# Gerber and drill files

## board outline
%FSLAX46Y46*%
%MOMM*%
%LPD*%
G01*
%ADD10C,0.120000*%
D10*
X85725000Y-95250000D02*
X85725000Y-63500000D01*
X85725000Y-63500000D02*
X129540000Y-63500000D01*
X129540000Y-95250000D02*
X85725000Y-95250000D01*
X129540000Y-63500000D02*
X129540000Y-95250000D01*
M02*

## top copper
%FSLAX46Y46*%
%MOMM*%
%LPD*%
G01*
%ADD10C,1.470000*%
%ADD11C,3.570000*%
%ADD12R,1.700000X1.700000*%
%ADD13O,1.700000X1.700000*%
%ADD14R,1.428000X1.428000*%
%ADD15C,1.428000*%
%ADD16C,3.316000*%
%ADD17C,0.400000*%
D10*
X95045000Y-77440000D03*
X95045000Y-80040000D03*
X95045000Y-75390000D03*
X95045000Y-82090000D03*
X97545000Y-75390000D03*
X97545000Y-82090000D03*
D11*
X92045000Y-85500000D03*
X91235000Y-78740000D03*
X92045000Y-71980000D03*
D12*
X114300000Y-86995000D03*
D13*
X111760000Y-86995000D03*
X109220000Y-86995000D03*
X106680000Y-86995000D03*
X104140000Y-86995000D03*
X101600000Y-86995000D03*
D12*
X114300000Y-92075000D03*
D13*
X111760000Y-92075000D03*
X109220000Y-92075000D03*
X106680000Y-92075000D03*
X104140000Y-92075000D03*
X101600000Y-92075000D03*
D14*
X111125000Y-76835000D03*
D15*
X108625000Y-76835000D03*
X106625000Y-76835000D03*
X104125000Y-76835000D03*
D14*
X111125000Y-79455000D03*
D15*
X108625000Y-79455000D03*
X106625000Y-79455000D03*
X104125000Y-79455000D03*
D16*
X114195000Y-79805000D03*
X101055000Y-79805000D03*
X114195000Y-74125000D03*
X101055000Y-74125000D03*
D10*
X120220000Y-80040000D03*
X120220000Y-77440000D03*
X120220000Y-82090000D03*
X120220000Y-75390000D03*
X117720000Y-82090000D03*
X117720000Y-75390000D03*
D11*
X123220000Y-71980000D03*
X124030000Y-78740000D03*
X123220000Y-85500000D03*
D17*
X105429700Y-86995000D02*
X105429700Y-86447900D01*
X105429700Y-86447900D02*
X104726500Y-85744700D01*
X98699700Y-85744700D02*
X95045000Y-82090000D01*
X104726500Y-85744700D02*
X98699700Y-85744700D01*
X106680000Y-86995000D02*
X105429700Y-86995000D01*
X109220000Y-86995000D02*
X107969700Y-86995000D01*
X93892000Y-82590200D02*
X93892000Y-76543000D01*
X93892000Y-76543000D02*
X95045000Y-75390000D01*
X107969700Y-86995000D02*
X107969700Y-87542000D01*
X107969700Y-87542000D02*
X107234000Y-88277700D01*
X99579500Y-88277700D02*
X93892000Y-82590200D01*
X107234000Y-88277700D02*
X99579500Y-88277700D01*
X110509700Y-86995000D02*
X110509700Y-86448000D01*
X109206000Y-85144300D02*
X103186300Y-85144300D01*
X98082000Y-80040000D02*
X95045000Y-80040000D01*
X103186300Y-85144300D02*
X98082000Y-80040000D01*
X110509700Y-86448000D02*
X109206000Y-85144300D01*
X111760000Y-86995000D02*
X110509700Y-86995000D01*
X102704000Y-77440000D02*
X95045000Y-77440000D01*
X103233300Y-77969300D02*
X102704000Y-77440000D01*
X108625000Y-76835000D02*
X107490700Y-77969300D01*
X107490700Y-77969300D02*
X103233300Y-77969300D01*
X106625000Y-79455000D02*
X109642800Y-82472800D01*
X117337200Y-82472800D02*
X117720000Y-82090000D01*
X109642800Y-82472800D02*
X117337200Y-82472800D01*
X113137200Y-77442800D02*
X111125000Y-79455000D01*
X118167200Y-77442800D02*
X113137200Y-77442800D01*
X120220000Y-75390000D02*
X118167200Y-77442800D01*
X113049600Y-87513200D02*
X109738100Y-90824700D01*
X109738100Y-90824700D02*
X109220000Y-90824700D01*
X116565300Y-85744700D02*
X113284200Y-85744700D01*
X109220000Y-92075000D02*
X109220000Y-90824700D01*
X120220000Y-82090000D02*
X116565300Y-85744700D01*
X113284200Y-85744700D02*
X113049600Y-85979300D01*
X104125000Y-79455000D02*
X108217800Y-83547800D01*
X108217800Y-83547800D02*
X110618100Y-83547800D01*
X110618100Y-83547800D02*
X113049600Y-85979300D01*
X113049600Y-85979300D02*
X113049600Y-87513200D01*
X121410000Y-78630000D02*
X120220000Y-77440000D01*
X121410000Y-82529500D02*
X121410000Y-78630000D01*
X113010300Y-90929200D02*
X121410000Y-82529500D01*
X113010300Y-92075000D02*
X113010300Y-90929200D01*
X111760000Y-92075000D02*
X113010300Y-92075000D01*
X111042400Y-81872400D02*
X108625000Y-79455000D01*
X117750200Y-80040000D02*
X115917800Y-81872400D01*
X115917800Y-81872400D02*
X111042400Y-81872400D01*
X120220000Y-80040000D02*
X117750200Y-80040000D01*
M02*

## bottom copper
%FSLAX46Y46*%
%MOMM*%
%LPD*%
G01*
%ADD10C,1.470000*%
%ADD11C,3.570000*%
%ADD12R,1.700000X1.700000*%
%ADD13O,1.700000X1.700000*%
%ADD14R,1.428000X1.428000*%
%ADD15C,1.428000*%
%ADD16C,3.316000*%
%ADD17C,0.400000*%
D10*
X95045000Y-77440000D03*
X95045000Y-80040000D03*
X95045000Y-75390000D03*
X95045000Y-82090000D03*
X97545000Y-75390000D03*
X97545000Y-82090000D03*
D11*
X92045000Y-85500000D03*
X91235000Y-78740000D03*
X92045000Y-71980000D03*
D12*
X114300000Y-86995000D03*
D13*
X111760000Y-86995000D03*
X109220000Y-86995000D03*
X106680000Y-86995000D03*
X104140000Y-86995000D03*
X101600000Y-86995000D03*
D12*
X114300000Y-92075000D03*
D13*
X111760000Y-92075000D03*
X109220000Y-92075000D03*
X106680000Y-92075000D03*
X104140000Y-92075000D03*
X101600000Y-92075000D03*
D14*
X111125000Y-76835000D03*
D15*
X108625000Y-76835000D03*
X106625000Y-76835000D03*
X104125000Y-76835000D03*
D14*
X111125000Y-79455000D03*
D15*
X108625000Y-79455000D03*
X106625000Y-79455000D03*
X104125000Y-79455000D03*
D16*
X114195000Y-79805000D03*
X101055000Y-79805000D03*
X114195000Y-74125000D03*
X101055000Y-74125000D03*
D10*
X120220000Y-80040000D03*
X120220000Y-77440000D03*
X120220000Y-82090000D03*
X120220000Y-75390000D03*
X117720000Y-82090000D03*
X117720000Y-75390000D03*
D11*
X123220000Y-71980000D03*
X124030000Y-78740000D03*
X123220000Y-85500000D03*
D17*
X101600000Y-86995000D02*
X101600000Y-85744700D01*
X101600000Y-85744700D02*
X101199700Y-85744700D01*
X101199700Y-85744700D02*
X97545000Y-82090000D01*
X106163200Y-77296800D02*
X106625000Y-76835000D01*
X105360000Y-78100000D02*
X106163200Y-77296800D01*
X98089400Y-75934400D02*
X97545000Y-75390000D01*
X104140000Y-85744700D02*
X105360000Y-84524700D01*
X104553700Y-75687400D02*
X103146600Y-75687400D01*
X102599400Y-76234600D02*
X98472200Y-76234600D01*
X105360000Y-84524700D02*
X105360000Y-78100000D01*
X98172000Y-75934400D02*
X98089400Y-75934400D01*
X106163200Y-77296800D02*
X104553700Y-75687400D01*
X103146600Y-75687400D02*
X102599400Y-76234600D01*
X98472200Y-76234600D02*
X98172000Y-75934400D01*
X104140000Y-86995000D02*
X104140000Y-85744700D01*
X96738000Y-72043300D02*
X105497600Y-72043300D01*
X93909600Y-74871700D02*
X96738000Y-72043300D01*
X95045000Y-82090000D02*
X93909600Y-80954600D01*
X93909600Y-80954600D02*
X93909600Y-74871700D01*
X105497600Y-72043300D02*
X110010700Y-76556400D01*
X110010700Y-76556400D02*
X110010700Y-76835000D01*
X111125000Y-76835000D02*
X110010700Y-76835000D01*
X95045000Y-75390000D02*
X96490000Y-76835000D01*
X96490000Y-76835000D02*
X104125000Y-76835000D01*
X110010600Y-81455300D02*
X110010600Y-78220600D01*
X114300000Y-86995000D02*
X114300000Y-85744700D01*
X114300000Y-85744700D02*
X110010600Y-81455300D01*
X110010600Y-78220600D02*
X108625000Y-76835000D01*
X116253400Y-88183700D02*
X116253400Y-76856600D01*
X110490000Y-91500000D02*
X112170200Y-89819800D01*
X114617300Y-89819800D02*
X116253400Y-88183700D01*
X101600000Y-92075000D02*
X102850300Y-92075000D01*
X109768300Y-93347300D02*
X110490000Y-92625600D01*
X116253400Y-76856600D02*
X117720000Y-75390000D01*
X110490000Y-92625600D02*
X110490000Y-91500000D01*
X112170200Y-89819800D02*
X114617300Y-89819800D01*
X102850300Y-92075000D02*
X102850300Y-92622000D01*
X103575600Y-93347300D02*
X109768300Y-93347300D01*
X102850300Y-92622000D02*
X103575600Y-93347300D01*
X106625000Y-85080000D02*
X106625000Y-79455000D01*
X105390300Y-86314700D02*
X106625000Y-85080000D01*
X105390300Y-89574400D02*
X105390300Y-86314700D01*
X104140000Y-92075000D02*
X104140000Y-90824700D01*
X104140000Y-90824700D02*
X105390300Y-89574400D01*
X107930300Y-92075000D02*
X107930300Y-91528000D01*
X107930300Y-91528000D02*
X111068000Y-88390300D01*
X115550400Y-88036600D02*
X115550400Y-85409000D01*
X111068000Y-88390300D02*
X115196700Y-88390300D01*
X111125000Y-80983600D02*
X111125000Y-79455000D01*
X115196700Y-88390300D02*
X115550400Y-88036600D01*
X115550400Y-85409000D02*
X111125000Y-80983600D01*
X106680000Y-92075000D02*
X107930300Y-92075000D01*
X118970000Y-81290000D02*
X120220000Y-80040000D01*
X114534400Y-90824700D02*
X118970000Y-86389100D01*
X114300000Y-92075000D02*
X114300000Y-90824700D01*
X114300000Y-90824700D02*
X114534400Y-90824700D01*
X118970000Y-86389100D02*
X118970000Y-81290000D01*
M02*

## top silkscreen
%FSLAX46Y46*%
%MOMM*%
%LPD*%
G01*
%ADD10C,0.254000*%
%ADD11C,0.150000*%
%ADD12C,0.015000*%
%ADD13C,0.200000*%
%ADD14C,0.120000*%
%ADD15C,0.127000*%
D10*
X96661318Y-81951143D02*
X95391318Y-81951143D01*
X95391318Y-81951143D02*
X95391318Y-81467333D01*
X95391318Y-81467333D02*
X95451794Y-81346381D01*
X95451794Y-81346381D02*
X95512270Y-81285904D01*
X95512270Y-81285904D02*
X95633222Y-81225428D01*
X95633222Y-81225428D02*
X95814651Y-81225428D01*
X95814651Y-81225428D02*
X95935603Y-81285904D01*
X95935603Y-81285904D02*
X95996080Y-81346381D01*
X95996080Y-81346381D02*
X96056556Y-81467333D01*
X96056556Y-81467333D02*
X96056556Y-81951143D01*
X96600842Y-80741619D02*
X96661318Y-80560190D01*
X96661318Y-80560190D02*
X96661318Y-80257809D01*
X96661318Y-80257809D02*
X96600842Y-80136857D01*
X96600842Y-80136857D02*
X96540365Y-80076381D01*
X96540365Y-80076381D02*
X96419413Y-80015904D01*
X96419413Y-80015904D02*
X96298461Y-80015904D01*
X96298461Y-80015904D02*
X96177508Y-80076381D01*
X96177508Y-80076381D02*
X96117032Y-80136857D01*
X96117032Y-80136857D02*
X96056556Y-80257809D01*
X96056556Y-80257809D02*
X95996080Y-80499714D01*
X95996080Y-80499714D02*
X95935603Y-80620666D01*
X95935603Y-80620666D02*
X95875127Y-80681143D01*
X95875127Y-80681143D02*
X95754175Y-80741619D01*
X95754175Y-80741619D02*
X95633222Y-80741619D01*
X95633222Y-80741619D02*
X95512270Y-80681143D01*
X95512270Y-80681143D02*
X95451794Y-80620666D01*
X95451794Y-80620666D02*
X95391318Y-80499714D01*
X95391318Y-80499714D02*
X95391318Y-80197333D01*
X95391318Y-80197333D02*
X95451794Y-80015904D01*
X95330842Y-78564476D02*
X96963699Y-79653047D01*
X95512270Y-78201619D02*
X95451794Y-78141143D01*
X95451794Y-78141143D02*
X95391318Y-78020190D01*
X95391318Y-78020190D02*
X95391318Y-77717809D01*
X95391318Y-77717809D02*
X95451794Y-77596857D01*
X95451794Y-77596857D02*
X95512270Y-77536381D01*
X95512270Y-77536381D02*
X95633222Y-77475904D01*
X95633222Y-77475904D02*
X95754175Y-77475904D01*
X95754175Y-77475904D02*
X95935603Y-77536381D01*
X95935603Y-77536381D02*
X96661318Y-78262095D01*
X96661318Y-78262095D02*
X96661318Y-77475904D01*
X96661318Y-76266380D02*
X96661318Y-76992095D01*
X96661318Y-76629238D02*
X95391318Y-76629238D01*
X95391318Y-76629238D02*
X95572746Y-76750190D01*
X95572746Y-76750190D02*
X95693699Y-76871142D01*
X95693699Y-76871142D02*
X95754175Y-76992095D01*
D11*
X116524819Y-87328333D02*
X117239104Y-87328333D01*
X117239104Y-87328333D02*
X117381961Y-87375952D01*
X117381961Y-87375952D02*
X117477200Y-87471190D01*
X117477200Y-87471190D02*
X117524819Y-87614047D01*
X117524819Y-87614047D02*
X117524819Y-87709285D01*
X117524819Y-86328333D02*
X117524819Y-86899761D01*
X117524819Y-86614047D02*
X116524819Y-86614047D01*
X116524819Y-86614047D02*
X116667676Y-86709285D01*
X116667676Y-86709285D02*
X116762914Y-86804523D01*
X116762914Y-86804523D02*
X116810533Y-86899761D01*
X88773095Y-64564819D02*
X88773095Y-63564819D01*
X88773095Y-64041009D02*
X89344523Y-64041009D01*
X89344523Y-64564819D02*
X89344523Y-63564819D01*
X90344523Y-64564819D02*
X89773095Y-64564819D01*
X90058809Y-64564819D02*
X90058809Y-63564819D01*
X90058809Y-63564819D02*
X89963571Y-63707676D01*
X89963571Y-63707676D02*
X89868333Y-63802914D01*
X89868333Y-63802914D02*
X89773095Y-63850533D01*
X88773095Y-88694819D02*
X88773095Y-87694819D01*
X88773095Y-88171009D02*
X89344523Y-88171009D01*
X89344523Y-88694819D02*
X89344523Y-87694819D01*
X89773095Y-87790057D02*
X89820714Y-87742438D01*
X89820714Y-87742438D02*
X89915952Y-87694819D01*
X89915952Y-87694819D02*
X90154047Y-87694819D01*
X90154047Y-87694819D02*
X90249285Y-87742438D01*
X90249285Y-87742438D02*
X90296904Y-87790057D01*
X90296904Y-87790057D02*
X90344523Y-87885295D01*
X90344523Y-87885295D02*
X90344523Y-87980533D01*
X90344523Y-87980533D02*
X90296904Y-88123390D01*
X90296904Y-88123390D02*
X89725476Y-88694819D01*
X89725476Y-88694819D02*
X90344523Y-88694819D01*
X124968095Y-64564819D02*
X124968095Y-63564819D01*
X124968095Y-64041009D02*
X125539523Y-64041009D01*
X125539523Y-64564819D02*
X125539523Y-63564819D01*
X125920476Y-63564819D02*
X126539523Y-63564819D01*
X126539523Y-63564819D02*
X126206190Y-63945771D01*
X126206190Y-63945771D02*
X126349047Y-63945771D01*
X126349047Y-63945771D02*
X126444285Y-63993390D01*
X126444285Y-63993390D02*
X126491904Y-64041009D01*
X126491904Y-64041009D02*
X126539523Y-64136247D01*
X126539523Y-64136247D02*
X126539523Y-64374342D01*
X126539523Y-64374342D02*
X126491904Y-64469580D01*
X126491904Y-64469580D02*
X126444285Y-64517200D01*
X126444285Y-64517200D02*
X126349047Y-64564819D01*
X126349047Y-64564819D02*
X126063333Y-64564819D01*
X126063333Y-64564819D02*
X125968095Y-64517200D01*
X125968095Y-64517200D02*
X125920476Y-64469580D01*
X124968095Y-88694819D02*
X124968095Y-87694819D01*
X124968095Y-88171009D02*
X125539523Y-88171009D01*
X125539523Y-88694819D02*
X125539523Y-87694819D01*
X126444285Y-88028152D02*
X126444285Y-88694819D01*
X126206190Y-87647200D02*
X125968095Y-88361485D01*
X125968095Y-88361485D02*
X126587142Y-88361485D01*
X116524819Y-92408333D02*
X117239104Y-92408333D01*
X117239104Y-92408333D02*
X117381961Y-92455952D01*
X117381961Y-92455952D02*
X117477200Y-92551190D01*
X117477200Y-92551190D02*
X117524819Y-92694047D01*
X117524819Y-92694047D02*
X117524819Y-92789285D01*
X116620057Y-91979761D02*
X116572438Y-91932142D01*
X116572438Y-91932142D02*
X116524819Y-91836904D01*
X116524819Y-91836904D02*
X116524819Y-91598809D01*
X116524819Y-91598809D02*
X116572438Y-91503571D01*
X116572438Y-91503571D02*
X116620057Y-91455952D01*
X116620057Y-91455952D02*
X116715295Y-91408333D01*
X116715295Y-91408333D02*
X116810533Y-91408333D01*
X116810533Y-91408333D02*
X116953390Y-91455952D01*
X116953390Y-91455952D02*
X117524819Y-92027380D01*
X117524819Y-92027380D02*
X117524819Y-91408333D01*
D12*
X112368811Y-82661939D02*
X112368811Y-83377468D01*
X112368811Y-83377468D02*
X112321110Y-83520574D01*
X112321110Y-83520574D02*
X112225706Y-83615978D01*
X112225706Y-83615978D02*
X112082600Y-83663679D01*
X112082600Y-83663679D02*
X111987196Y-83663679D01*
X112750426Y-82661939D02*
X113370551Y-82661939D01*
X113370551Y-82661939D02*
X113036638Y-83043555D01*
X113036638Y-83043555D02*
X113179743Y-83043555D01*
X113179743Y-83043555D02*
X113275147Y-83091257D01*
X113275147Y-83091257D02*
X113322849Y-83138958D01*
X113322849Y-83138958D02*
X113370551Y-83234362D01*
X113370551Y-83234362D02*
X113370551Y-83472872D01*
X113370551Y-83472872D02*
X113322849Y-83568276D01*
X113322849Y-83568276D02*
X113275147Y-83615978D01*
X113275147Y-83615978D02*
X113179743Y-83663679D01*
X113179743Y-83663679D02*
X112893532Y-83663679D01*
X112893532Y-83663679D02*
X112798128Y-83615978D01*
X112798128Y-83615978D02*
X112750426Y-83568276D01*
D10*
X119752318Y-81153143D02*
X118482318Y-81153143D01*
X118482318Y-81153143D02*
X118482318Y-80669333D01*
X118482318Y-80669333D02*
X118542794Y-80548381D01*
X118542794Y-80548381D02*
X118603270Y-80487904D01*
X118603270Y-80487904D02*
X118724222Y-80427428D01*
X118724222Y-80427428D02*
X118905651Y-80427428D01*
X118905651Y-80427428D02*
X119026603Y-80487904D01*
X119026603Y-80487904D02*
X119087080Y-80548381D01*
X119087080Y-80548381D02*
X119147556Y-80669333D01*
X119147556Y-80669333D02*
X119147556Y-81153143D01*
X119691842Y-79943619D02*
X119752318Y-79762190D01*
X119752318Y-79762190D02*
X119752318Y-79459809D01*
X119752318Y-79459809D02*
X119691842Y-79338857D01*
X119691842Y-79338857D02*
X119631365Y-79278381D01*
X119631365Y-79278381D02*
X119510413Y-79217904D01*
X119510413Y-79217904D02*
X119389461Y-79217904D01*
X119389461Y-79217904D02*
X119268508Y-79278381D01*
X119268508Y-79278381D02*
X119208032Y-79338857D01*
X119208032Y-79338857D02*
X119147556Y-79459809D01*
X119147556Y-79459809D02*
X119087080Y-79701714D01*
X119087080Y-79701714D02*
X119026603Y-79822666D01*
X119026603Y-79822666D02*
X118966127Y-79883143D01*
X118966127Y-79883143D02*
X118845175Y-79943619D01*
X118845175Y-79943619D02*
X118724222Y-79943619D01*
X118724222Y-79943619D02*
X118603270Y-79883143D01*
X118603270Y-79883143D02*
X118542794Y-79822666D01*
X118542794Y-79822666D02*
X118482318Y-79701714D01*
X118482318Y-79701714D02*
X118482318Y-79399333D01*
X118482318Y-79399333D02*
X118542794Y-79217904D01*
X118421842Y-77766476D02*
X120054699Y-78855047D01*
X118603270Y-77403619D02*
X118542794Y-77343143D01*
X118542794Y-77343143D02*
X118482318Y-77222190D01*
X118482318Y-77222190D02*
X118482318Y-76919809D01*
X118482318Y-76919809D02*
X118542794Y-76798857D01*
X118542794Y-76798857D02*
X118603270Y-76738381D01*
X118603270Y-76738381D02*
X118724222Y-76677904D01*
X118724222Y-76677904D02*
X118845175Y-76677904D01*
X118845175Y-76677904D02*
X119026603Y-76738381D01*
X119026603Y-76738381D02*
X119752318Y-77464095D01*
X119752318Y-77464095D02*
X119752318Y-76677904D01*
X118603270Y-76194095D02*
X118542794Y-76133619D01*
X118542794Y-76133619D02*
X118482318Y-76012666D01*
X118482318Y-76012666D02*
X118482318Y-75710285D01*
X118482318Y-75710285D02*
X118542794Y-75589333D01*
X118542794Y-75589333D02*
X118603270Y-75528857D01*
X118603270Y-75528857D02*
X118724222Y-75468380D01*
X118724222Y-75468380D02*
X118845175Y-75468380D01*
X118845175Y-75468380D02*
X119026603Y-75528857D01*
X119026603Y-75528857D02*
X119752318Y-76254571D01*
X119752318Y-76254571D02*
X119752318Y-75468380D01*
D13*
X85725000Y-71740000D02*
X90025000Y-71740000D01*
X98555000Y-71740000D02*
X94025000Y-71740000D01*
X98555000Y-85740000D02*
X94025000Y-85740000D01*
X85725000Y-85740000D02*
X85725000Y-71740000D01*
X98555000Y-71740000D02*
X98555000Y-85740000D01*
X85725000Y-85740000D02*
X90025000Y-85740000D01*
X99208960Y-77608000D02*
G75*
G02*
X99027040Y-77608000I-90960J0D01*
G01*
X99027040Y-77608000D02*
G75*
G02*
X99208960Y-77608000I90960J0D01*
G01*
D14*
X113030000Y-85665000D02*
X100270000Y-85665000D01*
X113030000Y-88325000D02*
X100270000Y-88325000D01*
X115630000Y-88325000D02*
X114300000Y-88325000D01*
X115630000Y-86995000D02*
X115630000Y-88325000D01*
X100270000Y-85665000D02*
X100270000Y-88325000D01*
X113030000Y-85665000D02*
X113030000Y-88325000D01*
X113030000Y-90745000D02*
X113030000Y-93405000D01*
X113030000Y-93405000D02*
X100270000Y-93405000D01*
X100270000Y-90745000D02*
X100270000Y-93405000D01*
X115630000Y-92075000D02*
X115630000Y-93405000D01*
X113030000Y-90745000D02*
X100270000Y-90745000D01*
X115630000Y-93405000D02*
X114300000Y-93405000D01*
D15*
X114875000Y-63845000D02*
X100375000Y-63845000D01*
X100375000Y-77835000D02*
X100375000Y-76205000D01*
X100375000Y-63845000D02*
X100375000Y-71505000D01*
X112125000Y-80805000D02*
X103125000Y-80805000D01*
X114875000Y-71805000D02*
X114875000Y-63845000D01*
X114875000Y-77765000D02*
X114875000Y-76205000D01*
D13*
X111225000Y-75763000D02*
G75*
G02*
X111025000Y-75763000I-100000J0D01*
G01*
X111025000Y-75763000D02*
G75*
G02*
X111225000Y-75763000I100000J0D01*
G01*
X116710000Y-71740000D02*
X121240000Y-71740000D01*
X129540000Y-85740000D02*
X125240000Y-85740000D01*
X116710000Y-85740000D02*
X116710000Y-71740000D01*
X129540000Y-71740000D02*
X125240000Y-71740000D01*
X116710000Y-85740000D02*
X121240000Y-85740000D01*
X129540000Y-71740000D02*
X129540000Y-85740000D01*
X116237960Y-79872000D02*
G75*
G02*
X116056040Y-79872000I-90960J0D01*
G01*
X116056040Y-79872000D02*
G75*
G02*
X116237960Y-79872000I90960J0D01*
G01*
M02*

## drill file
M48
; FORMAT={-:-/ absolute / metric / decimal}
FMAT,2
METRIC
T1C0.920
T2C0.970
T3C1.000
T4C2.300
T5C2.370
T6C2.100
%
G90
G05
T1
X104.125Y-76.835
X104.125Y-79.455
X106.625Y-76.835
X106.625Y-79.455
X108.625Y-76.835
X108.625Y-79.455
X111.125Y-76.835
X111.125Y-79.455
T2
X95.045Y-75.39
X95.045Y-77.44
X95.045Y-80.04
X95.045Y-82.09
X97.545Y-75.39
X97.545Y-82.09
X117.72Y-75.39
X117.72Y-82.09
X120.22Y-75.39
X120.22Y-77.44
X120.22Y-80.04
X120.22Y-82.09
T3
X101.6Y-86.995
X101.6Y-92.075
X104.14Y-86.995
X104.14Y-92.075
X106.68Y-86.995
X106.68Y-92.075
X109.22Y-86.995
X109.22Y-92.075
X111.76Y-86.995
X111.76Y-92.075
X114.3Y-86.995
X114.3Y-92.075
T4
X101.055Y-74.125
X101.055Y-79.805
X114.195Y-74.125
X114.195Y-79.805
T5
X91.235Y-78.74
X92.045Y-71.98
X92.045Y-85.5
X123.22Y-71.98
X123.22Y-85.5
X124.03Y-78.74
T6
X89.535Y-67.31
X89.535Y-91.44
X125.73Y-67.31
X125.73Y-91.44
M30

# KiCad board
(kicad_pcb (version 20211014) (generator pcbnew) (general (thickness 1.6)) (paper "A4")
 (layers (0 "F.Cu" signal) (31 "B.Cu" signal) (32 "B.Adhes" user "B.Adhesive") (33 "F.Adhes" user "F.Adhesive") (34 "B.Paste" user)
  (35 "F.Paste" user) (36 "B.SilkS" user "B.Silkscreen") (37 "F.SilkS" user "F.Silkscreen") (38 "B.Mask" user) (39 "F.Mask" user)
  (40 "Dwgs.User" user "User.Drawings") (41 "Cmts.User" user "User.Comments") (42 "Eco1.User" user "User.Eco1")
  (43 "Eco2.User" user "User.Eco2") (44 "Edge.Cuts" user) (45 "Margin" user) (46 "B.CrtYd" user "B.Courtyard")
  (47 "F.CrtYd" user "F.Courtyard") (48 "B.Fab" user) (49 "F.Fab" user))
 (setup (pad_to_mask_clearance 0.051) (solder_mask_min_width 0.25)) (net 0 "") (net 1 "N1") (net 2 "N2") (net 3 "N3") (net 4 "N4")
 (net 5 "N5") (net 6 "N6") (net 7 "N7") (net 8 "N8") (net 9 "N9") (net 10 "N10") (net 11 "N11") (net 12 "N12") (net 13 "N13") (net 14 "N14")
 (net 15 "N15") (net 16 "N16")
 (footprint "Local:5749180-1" (layer "F.Cu") (at 85.725 78.74 90)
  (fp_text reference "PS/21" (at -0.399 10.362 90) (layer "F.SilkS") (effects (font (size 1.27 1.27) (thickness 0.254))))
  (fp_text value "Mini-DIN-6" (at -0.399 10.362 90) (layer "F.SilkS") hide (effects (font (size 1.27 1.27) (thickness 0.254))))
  (fp_line (start 7 0) (end 7 4.3) (layer "F.SilkS") (width 0.2))
  (fp_line (start 7 12.83) (end 7 8.3) (layer "F.SilkS") (width 0.2))
  (fp_line (start -7 12.83) (end -7 8.3) (layer "F.SilkS") (width 0.2))
  (fp_line (start -7 0) (end 7 0) (layer "F.SilkS") (width 0.2))
  (fp_line (start 7 12.83) (end -7 12.83) (layer "F.SilkS") (width 0.2))
  (fp_line (start -7 0) (end -7 4.3) (layer "F.SilkS") (width 0.2))
  (fp_circle (center 1.132 13.393) (end 1.132 13.48396) (layer "F.SilkS") (width 0.2) (fill none))
  (pad "1" thru_hole circle locked (at 1.3 9.32 90) (size 1.47 1.47) (drill 0.97) (layers *.Cu *.Mask) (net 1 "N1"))
  (pad "2" thru_hole circle locked (at -1.3 9.32 90) (size 1.47 1.47) (drill 0.97) (layers *.Cu *.Mask) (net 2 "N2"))
  (pad "3" thru_hole circle locked (at 3.35 9.32 90) (size 1.47 1.47) (drill 0.97) (layers *.Cu *.Mask) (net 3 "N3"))
  (pad "4" thru_hole circle locked (at -3.35 9.32 90) (size 1.47 1.47) (drill 0.97) (layers *.Cu *.Mask) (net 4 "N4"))
  (pad "5" thru_hole circle locked (at 3.35 11.82 90) (size 1.47 1.47) (drill 0.97) (layers *.Cu *.Mask) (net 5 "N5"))
  (pad "6" thru_hole circle locked (at -3.35 11.82 90) (size 1.47 1.47) (drill 0.97) (layers *.Cu *.Mask) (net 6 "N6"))
  (pad "7" thru_hole circle locked (at -6.76 6.32 90) (size 3.57 3.57) (drill 2.37) (layers *.Cu *.Mask))
  (pad "8" thru_hole circle locked (at 0 5.51 90) (size 3.57 3.57) (drill 2.37) (layers *.Cu *.Mask))
  (pad "9" thru_hole circle locked (at 6.76 6.32 90) (size 3.57 3.57) (drill 2.37) (layers *.Cu *.Mask)))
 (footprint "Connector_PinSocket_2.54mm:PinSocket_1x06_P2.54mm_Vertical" (layer "F.Cu") (at 114.3 86.995 -90)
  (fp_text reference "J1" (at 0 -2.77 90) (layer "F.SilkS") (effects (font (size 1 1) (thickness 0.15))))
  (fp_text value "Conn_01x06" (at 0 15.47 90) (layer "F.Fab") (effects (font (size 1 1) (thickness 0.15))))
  (fp_line (start -1.33 1.27) (end -1.33 14.03) (layer "F.SilkS") (width 0.12))
  (fp_line (start 1.33 1.27) (end 1.33 14.03) (layer "F.SilkS") (width 0.12))
  (fp_line (start 1.33 -1.33) (end 1.33 0) (layer "F.SilkS") (width 0.12))
  (fp_line (start 0 -1.33) (end 1.33 -1.33) (layer "F.SilkS") (width 0.12))
  (fp_line (start -1.33 14.03) (end 1.33 14.03) (layer "F.SilkS") (width 0.12))
  (fp_line (start -1.33 1.27) (end 1.33 1.27) (layer "F.SilkS") (width 0.12))
  (pad "1" thru_hole rect locked (at 0 0 270) (size 1.7 1.7) (drill 1) (layers *.Cu *.Mask) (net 1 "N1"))
  (pad "2" thru_hole oval locked (at 0 2.54 270) (size 1.7 1.7) (drill 1) (layers *.Cu *.Mask) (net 2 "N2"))
  (pad "3" thru_hole oval locked (at 0 5.08 270) (size 1.7 1.7) (drill 1) (layers *.Cu *.Mask) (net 3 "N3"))
  (pad "4" thru_hole oval locked (at 0 7.62 270) (size 1.7 1.7) (drill 1) (layers *.Cu *.Mask) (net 4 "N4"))
  (pad "5" thru_hole oval locked (at 0 10.16 270) (size 1.7 1.7) (drill 1) (layers *.Cu *.Mask) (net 5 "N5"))
  (pad "6" thru_hole oval locked (at 0 12.7 270) (size 1.7 1.7) (drill 1) (layers *.Cu *.Mask) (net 6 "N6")))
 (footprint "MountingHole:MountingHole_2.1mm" (layer "F.Cu") (at 89.535 67.31)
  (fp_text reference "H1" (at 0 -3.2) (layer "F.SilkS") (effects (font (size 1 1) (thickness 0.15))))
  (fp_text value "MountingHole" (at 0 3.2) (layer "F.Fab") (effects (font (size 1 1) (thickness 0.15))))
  (pad "" np_thru_hole circle locked (at 0 0) (size 2.1 2.1) (drill 2.1) (layers *.Cu *.Mask)))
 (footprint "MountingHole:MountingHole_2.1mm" (layer "F.Cu") (at 89.535 91.44)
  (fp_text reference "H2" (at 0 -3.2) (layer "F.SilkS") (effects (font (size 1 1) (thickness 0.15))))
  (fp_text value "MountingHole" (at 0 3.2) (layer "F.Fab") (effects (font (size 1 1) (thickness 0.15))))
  (pad "" np_thru_hole circle locked (at 0 0) (size 2.1 2.1) (drill 2.1) (layers *.Cu *.Mask)))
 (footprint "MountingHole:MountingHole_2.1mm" (layer "F.Cu") (at 125.73 67.31)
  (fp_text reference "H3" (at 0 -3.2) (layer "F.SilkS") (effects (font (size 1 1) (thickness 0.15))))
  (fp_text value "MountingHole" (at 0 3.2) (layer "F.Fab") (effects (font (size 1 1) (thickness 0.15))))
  (pad "" np_thru_hole circle locked (at 0 0) (size 2.1 2.1) (drill 2.1) (layers *.Cu *.Mask)))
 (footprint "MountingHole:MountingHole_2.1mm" (layer "F.Cu") (at 125.73 91.44)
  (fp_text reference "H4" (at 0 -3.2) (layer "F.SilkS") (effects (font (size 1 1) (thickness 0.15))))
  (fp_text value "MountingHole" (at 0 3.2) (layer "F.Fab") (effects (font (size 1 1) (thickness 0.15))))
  (pad "" np_thru_hole circle locked (at 0 0) (size 2.1 2.1) (drill 2.1) (layers *.Cu *.Mask)))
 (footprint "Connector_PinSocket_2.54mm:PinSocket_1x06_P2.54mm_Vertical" (layer "F.Cu") (at 114.3 92.075 -90)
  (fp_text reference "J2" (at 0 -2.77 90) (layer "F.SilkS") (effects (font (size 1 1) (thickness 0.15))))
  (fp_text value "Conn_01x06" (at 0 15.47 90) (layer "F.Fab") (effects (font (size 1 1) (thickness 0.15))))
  (fp_line (start -1.33 1.27) (end 1.33 1.27) (layer "F.SilkS") (width 0.12))
  (fp_line (start 1.33 1.27) (end 1.33 14.03) (layer "F.SilkS") (width 0.12))
  (fp_line (start -1.33 14.03) (end 1.33 14.03) (layer "F.SilkS") (width 0.12))
  (fp_line (start 0 -1.33) (end 1.33 -1.33) (layer "F.SilkS") (width 0.12))
  (fp_line (start -1.33 1.27) (end -1.33 14.03) (layer "F.SilkS") (width 0.12))
  (fp_line (start 1.33 -1.33) (end 1.33 0) (layer "F.SilkS") (width 0.12))
  (pad "1" thru_hole rect locked (at 0 0 270) (size 1.7 1.7) (drill 1) (layers *.Cu *.Mask) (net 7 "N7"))
  (pad "2" thru_hole oval locked (at 0 2.54 270) (size 1.7 1.7) (drill 1) (layers *.Cu *.Mask) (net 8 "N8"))
  (pad "3" thru_hole oval locked (at 0 5.08 270) (size 1.7 1.7) (drill 1) (layers *.Cu *.Mask) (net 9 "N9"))
  (pad "4" thru_hole oval locked (at 0 7.62 270) (size 1.7 1.7) (drill 1) (layers *.Cu *.Mask) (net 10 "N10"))
  (pad "5" thru_hole oval locked (at 0 10.16 270) (size 1.7 1.7) (drill 1) (layers *.Cu *.Mask) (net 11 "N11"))
  (pad "6" thru_hole oval locked (at 0 12.7 270) (size 1.7 1.7) (drill 1) (layers *.Cu *.Mask) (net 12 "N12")))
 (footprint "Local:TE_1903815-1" (layer "F.Cu") (at 111.125 76.835 180)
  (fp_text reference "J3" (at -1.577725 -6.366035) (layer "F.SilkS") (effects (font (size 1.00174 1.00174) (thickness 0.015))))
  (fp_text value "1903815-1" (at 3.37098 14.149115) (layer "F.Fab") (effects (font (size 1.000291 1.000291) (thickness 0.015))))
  (fp_line (start -3.75 12.99) (end 10.75 12.99) (layer "F.SilkS") (width 0.127))
  (fp_line (start 10.75 -1) (end 10.75 0.63) (layer "F.SilkS") (width 0.127))
  (fp_line (start 10.75 12.99) (end 10.75 5.33) (layer "F.SilkS") (width 0.127))
  (fp_line (start -1 -3.97) (end 8 -3.97) (layer "F.SilkS") (width 0.127))
  (fp_line (start -3.75 5.03) (end -3.75 12.99) (layer "F.SilkS") (width 0.127))
  (fp_line (start -3.75 -0.93) (end -3.75 0.63) (layer "F.SilkS") (width 0.127))
  (fp_circle (center 0 1.072) (end 0.1 1.072) (layer "F.SilkS") (width 0.2) (fill none))
  (pad "1" thru_hole rect locked (at 0 0 180) (size 1.428 1.428) (drill 0.92) (layers *.Cu *.Mask) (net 4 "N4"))
  (pad "2" thru_hole circle locked (at 2.5 0 180) (size 1.428 1.428) (drill 0.92) (layers *.Cu *.Mask) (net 1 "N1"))
  (pad "3" thru_hole circle locked (at 4.5 0 180) (size 1.428 1.428) (drill 0.92) (layers *.Cu *.Mask) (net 5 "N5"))
  (pad "4" thru_hole circle locked (at 7 0 180) (size 1.428 1.428) (drill 0.92) (layers *.Cu *.Mask) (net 3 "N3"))
  (pad "5" thru_hole rect locked (at 0 -2.62 180) (size 1.428 1.428) (drill 0.92) (layers *.Cu *.Mask) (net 10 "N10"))
  (pad "6" thru_hole circle locked (at 2.5 -2.62 180) (size 1.428 1.428) (drill 0.92) (layers *.Cu *.Mask) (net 7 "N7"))
  (pad "7" thru_hole circle locked (at 4.5 -2.62 180) (size 1.428 1.428) (drill 0.92) (layers *.Cu *.Mask) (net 11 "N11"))
  (pad "8" thru_hole circle locked (at 7 -2.62 180) (size 1.428 1.428) (drill 0.92) (layers *.Cu *.Mask) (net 9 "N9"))
  (pad "P1" thru_hole circle locked (at -3.07 -2.97 180) (size 3.316 3.316) (drill 2.3) (layers *.Cu *.Mask) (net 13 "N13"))
  (pad "P2" thru_hole circle locked (at 10.07 -2.97 180) (size 3.316 3.316) (drill 2.3) (layers *.Cu *.Mask) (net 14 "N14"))
  (pad "P3" thru_hole circle locked (at -3.07 2.71 180) (size 3.316 3.316) (drill 2.3) (layers *.Cu *.Mask) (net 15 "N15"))
  (pad "P4" thru_hole circle locked (at 10.07 2.71 180) (size 3.316 3.316) (drill 2.3) (layers *.Cu *.Mask) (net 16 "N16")))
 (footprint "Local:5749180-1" (layer "F.Cu") (at 129.54 78.74 -90)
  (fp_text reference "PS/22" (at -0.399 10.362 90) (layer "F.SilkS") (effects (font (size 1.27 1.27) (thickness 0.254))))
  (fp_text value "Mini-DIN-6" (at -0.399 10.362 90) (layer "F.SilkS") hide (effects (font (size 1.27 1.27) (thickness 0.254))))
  (fp_line (start -7 12.83) (end -7 8.3) (layer "F.SilkS") (width 0.2))
  (fp_line (start 7 0) (end 7 4.3) (layer "F.SilkS") (width 0.2))
  (fp_line (start 7 12.83) (end -7 12.83) (layer "F.SilkS") (width 0.2))
  (fp_line (start -7 0) (end -7 4.3) (layer "F.SilkS") (width 0.2))
  (fp_line (start 7 12.83) (end 7 8.3) (layer "F.SilkS") (width 0.2))
  (fp_line (start -7 0) (end 7 0) (layer "F.SilkS") (width 0.2))
  (fp_circle (center 1.132 13.393) (end 1.132 13.48396) (layer "F.SilkS") (width 0.2) (fill none))
  (pad "1" thru_hole circle locked (at 1.3 9.32 270) (size 1.47 1.47) (drill 0.97) (layers *.Cu *.Mask) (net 7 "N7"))
  (pad "2" thru_hole circle locked (at -1.3 9.32 270) (size 1.47 1.47) (drill 0.97) (layers *.Cu *.Mask) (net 8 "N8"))
  (pad "3" thru_hole circle locked (at 3.35 9.32 270) (size 1.47 1.47) (drill 0.97) (layers *.Cu *.Mask) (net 9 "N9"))
  (pad "4" thru_hole circle locked (at -3.35 9.32 270) (size 1.47 1.47) (drill 0.97) (layers *.Cu *.Mask) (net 10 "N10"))
  (pad "5" thru_hole circle locked (at 3.35 11.82 270) (size 1.47 1.47) (drill 0.97) (layers *.Cu *.Mask) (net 11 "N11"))
  (pad "6" thru_hole circle locked (at -3.35 11.82 270) (size 1.47 1.47) (drill 0.97) (layers *.Cu *.Mask) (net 12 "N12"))
  (pad "7" thru_hole circle locked (at -6.76 6.32 270) (size 3.57 3.57) (drill 2.37) (layers *.Cu *.Mask))
  (pad "8" thru_hole circle locked (at 0 5.51 270) (size 3.57 3.57) (drill 2.37) (layers *.Cu *.Mask))
  (pad "9" thru_hole circle locked (at 6.76 6.32 270) (size 3.57 3.57) (drill 2.37) (layers *.Cu *.Mask)))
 (gr_line (start 85.725 95.25) (end 85.725 63.5) (layer "Edge.Cuts") (width 0.12))
 (gr_line (start 85.725 63.5) (end 129.54 63.5) (layer "Edge.Cuts") (width 0.12))
 (gr_line (start 129.54 95.25) (end 85.725 95.25) (layer "Edge.Cuts") (width 0.12))
 (gr_line (start 129.54 63.5) (end 129.54 95.25) (layer "Edge.Cuts") (width 0.12))
 (segment (start 101.6 86.995) (end 101.6 85.7447) (width 0.4) (layer "B.Cu") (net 6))
 (segment (start 101.6 85.7447) (end 101.1997 85.7447) (width 0.4) (layer "B.Cu") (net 6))
 (segment (start 101.1997 85.7447) (end 97.545 82.09) (width 0.4) (layer "B.Cu") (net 6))
 (segment (start 106.1632 77.2968) (end 106.625 76.835) (width 0.4) (layer "B.Cu") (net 5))
 (segment (start 105.36 78.1) (end 106.1632 77.2968) (width 0.4) (layer "B.Cu") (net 5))
 (segment (start 98.0894 75.9344) (end 97.545 75.39) (width 0.4) (layer "B.Cu") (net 5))
 (segment (start 104.14 85.7447) (end 105.36 84.5247) (width 0.4) (layer "B.Cu") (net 5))
 (segment (start 104.5537 75.6874) (end 103.1466 75.6874) (width 0.4) (layer "B.Cu") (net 5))
 (segment (start 102.5994 76.2346) (end 98.4722 76.2346) (width 0.4) (layer "B.Cu") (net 5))
 (segment (start 105.36 84.5247) (end 105.36 78.1) (width 0.4) (layer "B.Cu") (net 5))
 (segment (start 98.172 75.9344) (end 98.0894 75.9344) (width 0.4) (layer "B.Cu") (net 5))
 (segment (start 106.1632 77.2968) (end 104.5537 75.6874) (width 0.4) (layer "B.Cu") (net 5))
 (segment (start 103.1466 75.6874) (end 102.5994 76.2346) (width 0.4) (layer "B.Cu") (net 5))
 (segment (start 98.4722 76.2346) (end 98.172 75.9344) (width 0.4) (layer "B.Cu") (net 5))
 (segment (start 104.14 86.995) (end 104.14 85.7447) (width 0.4) (layer "B.Cu") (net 5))
 (segment (start 105.4297 86.995) (end 105.4297 86.4479) (width 0.4) (layer "F.Cu") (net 4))
 (segment (start 105.4297 86.4479) (end 104.7265 85.7447) (width 0.4) (layer "F.Cu") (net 4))
 (segment (start 98.6997 85.7447) (end 95.045 82.09) (width 0.4) (layer "F.Cu") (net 4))
 (segment (start 104.7265 85.7447) (end 98.6997 85.7447) (width 0.4) (layer "F.Cu") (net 4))
 (segment (start 106.68 86.995) (end 105.4297 86.995) (width 0.4) (layer "F.Cu") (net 4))
 (segment (start 96.738 72.0433) (end 105.4976 72.0433) (width 0.4) (layer "B.Cu") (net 4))
 (segment (start 93.9096 74.8717) (end 96.738 72.0433) (width 0.4) (layer "B.Cu") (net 4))
 (segment (start 95.045 82.09) (end 93.9096 80.9546) (width 0.4) (layer "B.Cu") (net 4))
 (segment (start 93.9096 80.9546) (end 93.9096 74.8717) (width 0.4) (layer "B.Cu") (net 4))
 (segment (start 105.4976 72.0433) (end 110.0107 76.5564) (width 0.4) (layer "B.Cu") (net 4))
 (segment (start 110.0107 76.5564) (end 110.0107 76.835) (width 0.4) (layer "B.Cu") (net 4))
 (segment (start 111.125 76.835) (end 110.0107 76.835) (width 0.4) (layer "B.Cu") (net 4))
 (segment (start 109.22 86.995) (end 107.9697 86.995) (width 0.4) (layer "F.Cu") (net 3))
 (segment (start 93.892 82.5902) (end 93.892 76.543) (width 0.4) (layer "F.Cu") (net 3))
 (segment (start 93.892 76.543) (end 95.045 75.39) (width 0.4) (layer "F.Cu") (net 3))
 (segment (start 107.9697 86.995) (end 107.9697 87.542) (width 0.4) (layer "F.Cu") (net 3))
 (segment (start 107.9697 87.542) (end 107.234 88.2777) (width 0.4) (layer "F.Cu") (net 3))
 (segment (start 99.5795 88.2777) (end 93.892 82.5902) (width 0.4) (layer "F.Cu") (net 3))
 (segment (start 107.234 88.2777) (end 99.5795 88.2777) (width 0.4) (layer "F.Cu") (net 3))
 (segment (start 95.045 75.39) (end 96.49 76.835) (width 0.4) (layer "B.Cu") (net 3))
 (segment (start 96.49 76.835) (end 104.125 76.835) (width 0.4) (layer "B.Cu") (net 3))
 (segment (start 110.5097 86.995) (end 110.5097 86.448) (width 0.4) (layer "F.Cu") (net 2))
 (segment (start 109.206 85.1443) (end 103.1863 85.1443) (width 0.4) (layer "F.Cu") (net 2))
 (segment (start 98.082 80.04) (end 95.045 80.04) (width 0.4) (layer "F.Cu") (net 2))
 (segment (start 103.1863 85.1443) (end 98.082 80.04) (width 0.4) (layer "F.Cu") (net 2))
 (segment (start 110.5097 86.448) (end 109.206 85.1443) (width 0.4) (layer "F.Cu") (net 2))
 (segment (start 111.76 86.995) (end 110.5097 86.995) (width 0.4) (layer "F.Cu") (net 2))
 (segment (start 102.704 77.44) (end 95.045 77.44) (width 0.4) (layer "F.Cu") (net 1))
 (segment (start 103.2333 77.9693) (end 102.704 77.44) (width 0.4) (layer "F.Cu") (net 1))
 (segment (start 108.625 76.835) (end 107.4907 77.9693) (width 0.4) (layer "F.Cu") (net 1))
 (segment (start 107.4907 77.9693) (end 103.2333 77.9693) (width 0.4) (layer "F.Cu") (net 1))
 (segment (start 110.0106 81.4553) (end 110.0106 78.2206) (width 0.4) (layer "B.Cu") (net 1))
 (segment (start 114.3 86.995) (end 114.3 85.7447) (width 0.4) (layer "B.Cu") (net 1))
 (segment (start 114.3 85.7447) (end 110.0106 81.4553) (width 0.4) (layer "B.Cu") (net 1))
 (segment (start 110.0106 78.2206) (end 108.625 76.835) (width 0.4) (layer "B.Cu") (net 1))
 (segment (start 116.2534 88.1837) (end 116.2534 76.8566) (width 0.4) (layer "B.Cu") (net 12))
 (segment (start 110.49 91.5) (end 112.1702 89.8198) (width 0.4) (layer "B.Cu") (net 12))
 (segment (start 114.6173 89.8198) (end 116.2534 88.1837) (width 0.4) (layer "B.Cu") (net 12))
 (segment (start 101.6 92.075) (end 102.8503 92.075) (width 0.4) (layer "B.Cu") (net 12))
 (segment (start 109.7683 93.3473) (end 110.49 92.6256) (width 0.4) (layer "B.Cu") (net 12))
 (segment (start 116.2534 76.8566) (end 117.72 75.39) (width 0.4) (layer "B.Cu") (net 12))
 (segment (start 110.49 92.6256) (end 110.49 91.5) (width 0.4) (layer "B.Cu") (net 12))
 (segment (start 112.1702 89.8198) (end 114.6173 89.8198) (width 0.4) (layer "B.Cu") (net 12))
 (segment (start 102.8503 92.075) (end 102.8503 92.622) (width 0.4) (layer "B.Cu") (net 12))
 (segment (start 103.5756 93.3473) (end 109.7683 93.3473) (width 0.4) (layer "B.Cu") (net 12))
 (segment (start 102.8503 92.622) (end 103.5756 93.3473) (width 0.4) (layer "B.Cu") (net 12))
 (segment (start 106.625 79.455) (end 109.6428 82.4728) (width 0.4) (layer "F.Cu") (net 11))
 (segment (start 117.3372 82.4728) (end 117.72 82.09) (width 0.4) (layer "F.Cu") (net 11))
 (segment (start 109.6428 82.4728) (end 117.3372 82.4728) (width 0.4) (layer "F.Cu") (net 11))
 (segment (start 106.625 85.08) (end 106.625 79.455) (width 0.4) (layer "B.Cu") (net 11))
 (segment (start 105.3903 86.3147) (end 106.625 85.08) (width 0.4) (layer "B.Cu") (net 11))
 (segment (start 105.3903 89.5744) (end 105.3903 86.3147) (width 0.4) (layer "B.Cu") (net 11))
 (segment (start 104.14 92.075) (end 104.14 90.8247) (width 0.4) (layer "B.Cu") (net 11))
 (segment (start 104.14 90.8247) (end 105.3903 89.5744) (width 0.4) (layer "B.Cu") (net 11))
 (segment (start 113.1372 77.4428) (end 111.125 79.455) (width 0.4) (layer "F.Cu") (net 10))
 (segment (start 118.1672 77.4428) (end 113.1372 77.4428) (width 0.4) (layer "F.Cu") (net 10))
 (segment (start 120.22 75.39) (end 118.1672 77.4428) (width 0.4) (layer "F.Cu") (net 10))
 (segment (start 107.9303 92.075) (end 107.9303 91.528) (width 0.4) (layer "B.Cu") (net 10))
 (segment (start 107.9303 91.528) (end 111.068 88.3903) (width 0.4) (layer "B.Cu") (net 10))
 (segment (start 115.5504 88.0366) (end 115.5504 85.409) (width 0.4) (layer "B.Cu") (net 10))
 (segment (start 111.068 88.3903) (end 115.1967 88.3903) (width 0.4) (layer "B.Cu") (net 10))
 (segment (start 111.125 80.9836) (end 111.125 79.455) (width 0.4) (layer "B.Cu") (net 10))
 (segment (start 115.1967 88.3903) (end 115.5504 88.0366) (width 0.4) (layer "B.Cu") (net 10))
 (segment (start 115.5504 85.409) (end 111.125 80.9836) (width 0.4) (layer "B.Cu") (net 10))
 (segment (start 106.68 92.075) (end 107.9303 92.075) (width 0.4) (layer "B.Cu") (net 10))
 (segment (start 113.0496 87.5132) (end 109.7381 90.8247) (width 0.4) (layer "F.Cu") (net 9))
 (segment (start 109.7381 90.8247) (end 109.22 90.8247) (width 0.4) (layer "F.Cu") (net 9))
 (segment (start 116.5653 85.7447) (end 113.2842 85.7447) (width 0.4) (layer "F.Cu") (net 9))
 (segment (start 109.22 92.075) (end 109.22 90.8247) (width 0.4) (layer "F.Cu") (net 9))
 (segment (start 120.22 82.09) (end 116.5653 85.7447) (width 0.4) (layer "F.Cu") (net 9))
 (segment (start 113.2842 85.7447) (end 113.0496 85.9793) (width 0.4) (layer "F.Cu") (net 9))
 (segment (start 104.125 79.455) (end 108.2178 83.5478) (width 0.4) (layer "F.Cu") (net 9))
 (segment (start 108.2178 83.5478) (end 110.6181 83.5478) (width 0.4) (layer "F.Cu") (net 9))
 (segment (start 110.6181 83.5478) (end 113.0496 85.9793) (width 0.4) (layer "F.Cu") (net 9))
 (segment (start 113.0496 85.9793) (end 113.0496 87.5132) (width 0.4) (layer "F.Cu") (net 9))
 (segment (start 121.41 78.63) (end 120.22 77.44) (width 0.4) (layer "F.Cu") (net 8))
 (segment (start 121.41 82.5295) (end 121.41 78.63) (width 0.4) (layer "F.Cu") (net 8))
 (segment (start 113.0103 90.9292) (end 121.41 82.5295) (width 0.4) (layer "F.Cu") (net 8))
 (segment (start 113.0103 92.075) (end 113.0103 90.9292) (width 0.4) (layer "F.Cu") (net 8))
 (segment (start 111.76 92.075) (end 113.0103 92.075) (width 0.4) (layer "F.Cu") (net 8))
 (segment (start 111.0424 81.8724) (end 108.625 79.455) (width 0.4) (layer "F.Cu") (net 7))
 (segment (start 117.7502 80.04) (end 115.9178 81.8724) (width 0.4) (layer "F.Cu") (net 7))
 (segment (start 115.9178 81.8724) (end 111.0424 81.8724) (width 0.4) (layer "F.Cu") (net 7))
 (segment (start 120.22 80.04) (end 117.7502 80.04) (width 0.4) (layer "F.Cu") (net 7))
 (segment (start 118.97 81.29) (end 120.22 80.04) (width 0.4) (layer "B.Cu") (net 7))
 (segment (start 114.5344 90.8247) (end 118.97 86.3891) (width 0.4) (layer "B.Cu") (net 7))
 (segment (start 114.3 92.075) (end 114.3 90.8247) (width 0.4) (layer "B.Cu") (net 7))
 (segment (start 114.3 90.8247) (end 114.5344 90.8247) (width 0.4) (layer "B.Cu") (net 7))
 (segment (start 118.97 86.3891) (end 118.97 81.29) (width 0.4) (layer "B.Cu") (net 7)))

